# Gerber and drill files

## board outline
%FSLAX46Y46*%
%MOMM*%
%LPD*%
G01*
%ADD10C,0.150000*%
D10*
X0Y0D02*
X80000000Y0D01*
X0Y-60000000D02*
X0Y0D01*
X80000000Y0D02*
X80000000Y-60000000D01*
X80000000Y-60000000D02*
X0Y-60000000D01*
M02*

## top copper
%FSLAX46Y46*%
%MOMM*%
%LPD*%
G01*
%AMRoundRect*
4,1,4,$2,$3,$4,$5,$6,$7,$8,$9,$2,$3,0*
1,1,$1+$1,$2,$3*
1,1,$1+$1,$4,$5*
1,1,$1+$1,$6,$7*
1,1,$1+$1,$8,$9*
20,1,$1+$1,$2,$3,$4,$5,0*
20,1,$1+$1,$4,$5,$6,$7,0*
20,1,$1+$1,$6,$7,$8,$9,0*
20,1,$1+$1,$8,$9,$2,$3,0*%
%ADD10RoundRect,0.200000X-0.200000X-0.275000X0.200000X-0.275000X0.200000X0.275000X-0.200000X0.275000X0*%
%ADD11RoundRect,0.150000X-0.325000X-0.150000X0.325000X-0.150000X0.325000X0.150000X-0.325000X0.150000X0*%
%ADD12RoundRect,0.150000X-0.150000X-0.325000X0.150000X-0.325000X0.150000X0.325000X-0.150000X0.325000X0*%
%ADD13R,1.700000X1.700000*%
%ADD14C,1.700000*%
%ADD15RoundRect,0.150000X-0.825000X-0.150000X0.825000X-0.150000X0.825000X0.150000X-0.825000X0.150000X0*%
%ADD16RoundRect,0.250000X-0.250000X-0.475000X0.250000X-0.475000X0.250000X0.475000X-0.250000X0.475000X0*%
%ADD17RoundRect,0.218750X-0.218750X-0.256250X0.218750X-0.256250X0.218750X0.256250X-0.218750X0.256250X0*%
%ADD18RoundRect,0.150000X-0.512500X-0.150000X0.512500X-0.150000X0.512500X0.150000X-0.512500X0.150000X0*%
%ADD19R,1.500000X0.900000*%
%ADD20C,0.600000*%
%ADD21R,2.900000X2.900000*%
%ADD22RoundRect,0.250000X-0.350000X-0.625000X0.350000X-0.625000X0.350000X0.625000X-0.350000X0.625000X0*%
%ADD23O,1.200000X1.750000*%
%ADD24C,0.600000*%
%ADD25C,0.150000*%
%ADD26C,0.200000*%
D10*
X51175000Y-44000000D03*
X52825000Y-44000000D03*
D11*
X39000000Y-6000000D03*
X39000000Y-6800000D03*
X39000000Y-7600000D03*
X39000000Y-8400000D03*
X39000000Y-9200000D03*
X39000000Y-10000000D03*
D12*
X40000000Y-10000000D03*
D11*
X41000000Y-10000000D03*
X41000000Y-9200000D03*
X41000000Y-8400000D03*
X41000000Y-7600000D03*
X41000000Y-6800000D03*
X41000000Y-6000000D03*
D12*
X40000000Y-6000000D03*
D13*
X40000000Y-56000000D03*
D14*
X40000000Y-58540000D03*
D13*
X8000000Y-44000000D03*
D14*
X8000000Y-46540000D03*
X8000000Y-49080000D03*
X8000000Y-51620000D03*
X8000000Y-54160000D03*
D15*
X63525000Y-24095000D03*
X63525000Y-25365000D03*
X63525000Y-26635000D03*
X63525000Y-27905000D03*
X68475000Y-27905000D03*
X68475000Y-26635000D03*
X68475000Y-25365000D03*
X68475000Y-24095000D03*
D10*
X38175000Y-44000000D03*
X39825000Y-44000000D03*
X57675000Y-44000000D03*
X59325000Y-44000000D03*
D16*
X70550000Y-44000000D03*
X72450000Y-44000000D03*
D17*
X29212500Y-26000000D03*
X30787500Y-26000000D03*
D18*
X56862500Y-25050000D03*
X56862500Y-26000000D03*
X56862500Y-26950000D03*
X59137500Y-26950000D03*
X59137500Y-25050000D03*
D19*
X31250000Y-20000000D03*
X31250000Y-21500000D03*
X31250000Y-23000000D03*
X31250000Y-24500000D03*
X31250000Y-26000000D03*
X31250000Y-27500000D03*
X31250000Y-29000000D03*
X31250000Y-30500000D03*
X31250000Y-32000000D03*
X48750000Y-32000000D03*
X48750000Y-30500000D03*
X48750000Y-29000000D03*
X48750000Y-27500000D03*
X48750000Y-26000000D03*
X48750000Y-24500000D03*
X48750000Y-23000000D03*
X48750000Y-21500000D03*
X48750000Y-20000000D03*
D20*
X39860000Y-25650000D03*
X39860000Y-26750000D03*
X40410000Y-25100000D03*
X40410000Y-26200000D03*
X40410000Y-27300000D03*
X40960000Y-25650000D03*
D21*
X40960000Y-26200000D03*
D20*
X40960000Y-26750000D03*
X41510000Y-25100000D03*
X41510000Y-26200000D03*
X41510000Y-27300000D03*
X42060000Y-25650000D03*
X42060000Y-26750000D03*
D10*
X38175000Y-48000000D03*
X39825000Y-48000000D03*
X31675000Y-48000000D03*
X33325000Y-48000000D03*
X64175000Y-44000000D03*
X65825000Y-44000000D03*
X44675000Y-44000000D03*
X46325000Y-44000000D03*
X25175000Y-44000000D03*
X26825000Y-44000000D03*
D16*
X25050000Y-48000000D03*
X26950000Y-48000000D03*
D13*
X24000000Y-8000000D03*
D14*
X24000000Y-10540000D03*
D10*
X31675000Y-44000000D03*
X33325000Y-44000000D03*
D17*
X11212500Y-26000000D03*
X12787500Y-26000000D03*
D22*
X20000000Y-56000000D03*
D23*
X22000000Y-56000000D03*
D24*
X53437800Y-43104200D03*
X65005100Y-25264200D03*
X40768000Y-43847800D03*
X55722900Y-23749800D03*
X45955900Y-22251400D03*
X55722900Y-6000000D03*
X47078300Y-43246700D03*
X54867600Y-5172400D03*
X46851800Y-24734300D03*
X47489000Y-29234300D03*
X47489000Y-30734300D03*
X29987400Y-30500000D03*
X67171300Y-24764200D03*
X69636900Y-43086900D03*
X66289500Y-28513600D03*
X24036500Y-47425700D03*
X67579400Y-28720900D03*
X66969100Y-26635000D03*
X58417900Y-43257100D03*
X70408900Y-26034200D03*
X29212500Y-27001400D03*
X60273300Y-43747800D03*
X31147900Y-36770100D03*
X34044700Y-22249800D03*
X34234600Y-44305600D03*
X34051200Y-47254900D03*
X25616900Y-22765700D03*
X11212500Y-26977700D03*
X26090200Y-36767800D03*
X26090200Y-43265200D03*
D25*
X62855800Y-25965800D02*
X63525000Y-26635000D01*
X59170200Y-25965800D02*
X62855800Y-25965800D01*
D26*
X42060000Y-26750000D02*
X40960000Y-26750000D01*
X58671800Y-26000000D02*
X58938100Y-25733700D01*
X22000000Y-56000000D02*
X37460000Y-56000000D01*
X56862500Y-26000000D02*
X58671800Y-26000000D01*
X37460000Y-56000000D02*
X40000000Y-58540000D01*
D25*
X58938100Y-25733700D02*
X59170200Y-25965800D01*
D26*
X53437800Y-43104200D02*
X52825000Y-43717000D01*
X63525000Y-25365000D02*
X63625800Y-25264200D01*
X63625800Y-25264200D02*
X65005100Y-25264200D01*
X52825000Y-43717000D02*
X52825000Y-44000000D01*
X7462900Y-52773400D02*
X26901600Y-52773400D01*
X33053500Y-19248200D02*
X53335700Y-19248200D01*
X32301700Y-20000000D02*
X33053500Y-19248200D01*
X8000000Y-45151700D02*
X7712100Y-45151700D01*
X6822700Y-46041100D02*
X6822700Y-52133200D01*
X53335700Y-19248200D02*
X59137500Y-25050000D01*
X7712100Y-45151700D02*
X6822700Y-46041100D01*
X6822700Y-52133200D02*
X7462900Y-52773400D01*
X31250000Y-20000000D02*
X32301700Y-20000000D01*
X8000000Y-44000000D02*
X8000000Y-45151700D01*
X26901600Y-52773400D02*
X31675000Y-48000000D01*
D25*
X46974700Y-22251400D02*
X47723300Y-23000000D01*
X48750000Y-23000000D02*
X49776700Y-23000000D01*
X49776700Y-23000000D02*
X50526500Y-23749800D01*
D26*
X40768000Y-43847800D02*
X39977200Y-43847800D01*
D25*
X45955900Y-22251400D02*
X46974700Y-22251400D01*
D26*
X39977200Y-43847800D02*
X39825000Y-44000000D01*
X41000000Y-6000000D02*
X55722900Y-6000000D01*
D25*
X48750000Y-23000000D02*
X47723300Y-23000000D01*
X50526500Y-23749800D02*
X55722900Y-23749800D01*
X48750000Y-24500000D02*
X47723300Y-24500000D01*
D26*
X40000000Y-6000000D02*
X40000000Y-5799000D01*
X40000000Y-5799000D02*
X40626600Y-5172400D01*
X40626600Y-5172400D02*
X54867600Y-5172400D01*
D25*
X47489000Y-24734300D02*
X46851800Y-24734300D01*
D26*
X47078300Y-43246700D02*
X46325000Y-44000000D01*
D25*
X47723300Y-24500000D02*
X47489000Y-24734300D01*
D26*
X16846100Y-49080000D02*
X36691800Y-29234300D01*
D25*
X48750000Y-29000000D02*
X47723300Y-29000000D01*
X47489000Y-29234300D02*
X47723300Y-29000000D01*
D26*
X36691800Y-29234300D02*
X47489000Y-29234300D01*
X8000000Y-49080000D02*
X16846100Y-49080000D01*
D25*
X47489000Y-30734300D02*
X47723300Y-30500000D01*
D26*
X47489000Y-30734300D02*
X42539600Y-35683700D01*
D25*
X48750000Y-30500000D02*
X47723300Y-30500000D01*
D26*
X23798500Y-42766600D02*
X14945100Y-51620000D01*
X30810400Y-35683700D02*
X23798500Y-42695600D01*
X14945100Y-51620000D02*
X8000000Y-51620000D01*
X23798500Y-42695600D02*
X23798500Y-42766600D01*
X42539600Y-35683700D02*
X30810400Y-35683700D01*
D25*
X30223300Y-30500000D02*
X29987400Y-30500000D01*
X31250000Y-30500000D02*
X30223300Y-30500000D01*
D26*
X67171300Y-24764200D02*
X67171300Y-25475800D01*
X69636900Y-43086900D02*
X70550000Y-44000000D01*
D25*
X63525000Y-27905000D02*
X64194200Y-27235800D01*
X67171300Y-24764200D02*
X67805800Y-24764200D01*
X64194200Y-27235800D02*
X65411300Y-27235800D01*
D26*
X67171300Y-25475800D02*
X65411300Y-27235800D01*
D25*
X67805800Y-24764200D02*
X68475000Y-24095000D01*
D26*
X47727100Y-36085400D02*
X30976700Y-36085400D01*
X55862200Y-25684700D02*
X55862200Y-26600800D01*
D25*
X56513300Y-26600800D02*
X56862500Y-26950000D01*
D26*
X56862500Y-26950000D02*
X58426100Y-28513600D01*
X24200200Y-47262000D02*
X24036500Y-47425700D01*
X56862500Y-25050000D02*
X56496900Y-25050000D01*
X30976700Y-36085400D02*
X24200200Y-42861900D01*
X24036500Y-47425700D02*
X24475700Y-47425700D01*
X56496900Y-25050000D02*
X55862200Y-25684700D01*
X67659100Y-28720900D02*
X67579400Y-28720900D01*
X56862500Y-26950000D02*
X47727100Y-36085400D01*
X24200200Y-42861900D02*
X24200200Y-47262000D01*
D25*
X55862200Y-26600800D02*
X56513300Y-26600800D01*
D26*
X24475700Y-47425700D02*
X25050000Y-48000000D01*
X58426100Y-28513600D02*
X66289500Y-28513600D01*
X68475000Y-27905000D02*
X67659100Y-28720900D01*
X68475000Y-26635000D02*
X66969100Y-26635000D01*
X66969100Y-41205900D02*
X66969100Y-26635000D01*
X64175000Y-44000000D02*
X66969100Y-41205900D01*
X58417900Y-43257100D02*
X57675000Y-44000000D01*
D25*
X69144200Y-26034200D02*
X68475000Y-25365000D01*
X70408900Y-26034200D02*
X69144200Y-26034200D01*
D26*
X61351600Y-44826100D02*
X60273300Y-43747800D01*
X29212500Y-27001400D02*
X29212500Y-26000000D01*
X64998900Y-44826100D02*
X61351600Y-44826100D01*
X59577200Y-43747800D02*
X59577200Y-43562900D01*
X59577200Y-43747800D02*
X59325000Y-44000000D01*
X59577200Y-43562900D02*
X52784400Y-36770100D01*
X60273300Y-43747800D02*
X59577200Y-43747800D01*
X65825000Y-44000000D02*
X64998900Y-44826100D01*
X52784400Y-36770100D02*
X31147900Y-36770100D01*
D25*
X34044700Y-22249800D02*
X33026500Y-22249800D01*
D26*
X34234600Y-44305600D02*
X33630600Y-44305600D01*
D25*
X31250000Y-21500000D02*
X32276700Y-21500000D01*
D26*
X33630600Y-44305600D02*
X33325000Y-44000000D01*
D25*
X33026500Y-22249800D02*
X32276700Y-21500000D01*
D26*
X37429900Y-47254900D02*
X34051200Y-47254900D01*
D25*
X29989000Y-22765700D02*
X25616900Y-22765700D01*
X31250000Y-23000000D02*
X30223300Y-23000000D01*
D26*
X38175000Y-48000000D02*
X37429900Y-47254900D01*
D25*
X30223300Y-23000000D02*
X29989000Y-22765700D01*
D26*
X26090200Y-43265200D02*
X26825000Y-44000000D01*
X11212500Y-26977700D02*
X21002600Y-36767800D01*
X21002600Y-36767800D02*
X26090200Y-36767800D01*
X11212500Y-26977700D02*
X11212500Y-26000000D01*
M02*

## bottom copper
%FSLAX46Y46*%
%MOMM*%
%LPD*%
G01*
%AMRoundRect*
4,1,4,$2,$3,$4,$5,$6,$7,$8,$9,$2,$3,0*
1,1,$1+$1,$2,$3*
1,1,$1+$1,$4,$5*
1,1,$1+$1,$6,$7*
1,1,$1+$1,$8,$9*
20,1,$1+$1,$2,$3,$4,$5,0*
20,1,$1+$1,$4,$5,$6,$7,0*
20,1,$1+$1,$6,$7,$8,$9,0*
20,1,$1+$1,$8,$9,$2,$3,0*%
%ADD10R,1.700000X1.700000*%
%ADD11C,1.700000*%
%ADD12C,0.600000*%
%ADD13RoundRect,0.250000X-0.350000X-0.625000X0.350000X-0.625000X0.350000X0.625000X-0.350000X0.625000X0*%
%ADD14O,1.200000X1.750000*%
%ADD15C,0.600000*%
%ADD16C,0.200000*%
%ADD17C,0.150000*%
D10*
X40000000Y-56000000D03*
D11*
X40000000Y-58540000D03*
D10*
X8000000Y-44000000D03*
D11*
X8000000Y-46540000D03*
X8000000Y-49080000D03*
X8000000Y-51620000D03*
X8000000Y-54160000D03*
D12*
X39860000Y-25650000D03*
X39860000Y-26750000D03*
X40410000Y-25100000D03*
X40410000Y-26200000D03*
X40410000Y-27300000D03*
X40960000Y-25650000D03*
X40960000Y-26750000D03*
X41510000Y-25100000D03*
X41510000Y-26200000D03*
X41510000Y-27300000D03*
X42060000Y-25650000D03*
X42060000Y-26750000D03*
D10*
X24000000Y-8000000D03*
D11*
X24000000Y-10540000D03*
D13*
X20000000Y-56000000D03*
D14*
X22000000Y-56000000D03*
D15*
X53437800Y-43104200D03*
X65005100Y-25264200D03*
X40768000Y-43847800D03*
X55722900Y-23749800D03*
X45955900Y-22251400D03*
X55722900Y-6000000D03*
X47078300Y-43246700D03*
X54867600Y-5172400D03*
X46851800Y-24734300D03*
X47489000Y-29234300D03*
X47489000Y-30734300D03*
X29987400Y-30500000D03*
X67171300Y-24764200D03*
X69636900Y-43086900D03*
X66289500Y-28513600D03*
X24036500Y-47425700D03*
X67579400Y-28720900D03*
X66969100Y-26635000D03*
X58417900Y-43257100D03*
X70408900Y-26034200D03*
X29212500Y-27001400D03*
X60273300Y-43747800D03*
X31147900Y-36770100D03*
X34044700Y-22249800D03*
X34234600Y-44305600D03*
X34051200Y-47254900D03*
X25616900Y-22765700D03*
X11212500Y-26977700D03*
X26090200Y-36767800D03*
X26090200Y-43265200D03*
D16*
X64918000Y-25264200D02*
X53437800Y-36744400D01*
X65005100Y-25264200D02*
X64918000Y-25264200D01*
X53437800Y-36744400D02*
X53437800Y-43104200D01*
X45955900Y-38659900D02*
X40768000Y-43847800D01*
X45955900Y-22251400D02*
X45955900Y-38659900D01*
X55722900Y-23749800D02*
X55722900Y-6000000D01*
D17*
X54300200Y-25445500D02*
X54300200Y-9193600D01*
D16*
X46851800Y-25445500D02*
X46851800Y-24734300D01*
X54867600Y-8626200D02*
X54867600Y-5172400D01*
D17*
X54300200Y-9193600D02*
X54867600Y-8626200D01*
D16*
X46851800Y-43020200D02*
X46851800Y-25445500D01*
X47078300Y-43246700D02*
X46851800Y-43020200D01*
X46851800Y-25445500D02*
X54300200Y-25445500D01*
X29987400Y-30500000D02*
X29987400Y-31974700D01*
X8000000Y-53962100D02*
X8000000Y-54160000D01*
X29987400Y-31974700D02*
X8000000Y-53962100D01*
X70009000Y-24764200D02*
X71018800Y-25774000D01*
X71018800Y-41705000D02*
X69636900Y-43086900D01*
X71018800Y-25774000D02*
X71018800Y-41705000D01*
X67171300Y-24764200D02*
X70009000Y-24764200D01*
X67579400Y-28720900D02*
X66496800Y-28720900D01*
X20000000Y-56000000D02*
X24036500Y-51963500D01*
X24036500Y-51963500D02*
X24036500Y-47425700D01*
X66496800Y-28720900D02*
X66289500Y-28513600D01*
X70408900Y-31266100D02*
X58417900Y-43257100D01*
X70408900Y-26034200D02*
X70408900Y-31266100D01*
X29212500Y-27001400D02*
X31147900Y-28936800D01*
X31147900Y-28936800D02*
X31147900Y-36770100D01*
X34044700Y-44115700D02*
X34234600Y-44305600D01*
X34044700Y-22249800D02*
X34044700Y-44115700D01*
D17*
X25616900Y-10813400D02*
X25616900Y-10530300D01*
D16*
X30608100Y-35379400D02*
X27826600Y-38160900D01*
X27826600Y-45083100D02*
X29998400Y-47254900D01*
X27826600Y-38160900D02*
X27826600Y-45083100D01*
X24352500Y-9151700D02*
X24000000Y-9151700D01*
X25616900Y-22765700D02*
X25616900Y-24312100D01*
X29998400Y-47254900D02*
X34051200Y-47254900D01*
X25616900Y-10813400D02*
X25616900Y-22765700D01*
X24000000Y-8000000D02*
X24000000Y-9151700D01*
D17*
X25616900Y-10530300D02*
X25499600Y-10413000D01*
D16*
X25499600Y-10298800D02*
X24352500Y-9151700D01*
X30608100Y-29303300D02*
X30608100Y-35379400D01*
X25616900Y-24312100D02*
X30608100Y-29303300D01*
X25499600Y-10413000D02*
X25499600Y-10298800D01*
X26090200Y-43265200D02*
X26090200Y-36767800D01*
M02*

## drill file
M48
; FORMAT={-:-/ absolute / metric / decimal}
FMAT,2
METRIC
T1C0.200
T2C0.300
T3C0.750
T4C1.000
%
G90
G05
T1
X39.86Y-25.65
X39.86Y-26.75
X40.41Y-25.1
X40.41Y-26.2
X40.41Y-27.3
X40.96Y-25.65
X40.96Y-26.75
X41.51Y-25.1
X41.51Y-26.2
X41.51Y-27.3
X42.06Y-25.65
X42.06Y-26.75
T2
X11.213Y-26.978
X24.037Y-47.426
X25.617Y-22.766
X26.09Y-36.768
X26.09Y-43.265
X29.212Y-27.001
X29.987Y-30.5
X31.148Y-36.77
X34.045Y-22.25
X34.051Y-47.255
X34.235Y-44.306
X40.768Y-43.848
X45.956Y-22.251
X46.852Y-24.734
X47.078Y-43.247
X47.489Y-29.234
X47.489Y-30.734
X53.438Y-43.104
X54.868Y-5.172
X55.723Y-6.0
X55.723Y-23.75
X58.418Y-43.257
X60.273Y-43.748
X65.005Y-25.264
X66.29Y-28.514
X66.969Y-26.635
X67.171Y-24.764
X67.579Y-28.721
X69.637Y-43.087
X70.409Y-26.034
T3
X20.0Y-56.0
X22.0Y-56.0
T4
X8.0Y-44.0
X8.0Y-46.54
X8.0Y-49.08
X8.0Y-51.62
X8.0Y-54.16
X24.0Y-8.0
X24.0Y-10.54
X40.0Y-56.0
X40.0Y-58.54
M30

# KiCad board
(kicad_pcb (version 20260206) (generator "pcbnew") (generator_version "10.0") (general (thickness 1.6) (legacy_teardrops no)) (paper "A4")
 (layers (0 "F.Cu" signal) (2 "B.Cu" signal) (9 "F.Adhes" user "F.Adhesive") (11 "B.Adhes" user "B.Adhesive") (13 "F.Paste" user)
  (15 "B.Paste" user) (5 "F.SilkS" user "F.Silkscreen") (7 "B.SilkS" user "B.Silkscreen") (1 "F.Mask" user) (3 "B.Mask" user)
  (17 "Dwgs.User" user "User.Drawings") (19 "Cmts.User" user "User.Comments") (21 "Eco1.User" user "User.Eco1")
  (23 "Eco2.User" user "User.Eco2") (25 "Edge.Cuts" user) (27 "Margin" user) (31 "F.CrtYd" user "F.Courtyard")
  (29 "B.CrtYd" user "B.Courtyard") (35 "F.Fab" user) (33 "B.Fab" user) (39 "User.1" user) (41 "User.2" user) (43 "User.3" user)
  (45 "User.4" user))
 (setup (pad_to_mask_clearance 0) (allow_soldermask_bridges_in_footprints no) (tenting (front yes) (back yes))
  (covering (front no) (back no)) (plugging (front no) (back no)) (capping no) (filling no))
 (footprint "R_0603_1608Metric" (layer "F.Cu") (at 52 44)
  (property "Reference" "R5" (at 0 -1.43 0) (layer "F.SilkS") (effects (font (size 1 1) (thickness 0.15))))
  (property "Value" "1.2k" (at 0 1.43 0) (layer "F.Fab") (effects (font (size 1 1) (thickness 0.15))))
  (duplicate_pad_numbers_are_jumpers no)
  (pad "1" smd roundrect (at -0.825 0) (size 0.8 0.95) (layers "F.Cu" "F.Mask" "F.Paste") (roundrect_rratio 0.25) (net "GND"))
  (pad "2" smd roundrect (at 0.825 0) (size 0.8 0.95) (layers "F.Cu" "F.Mask" "F.Paste") (roundrect_rratio 0.25) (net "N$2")))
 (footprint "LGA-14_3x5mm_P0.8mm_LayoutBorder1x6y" (layer "F.Cu") (at 40 8)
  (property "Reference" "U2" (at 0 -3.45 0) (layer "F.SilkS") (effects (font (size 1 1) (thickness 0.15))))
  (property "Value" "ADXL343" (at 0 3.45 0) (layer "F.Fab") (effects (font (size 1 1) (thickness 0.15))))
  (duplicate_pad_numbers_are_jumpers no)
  (pad "1" smd roundrect (at -1 -2) (size 0.95 0.6) (layers "F.Cu" "F.Mask" "F.Paste") (roundrect_rratio 0.25) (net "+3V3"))
  (pad "2" smd roundrect (at -1 -1.2) (size 0.95 0.6) (layers "F.Cu" "F.Mask" "F.Paste") (roundrect_rratio 0.25) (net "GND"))
  (pad "3" smd roundrect (at -1 -0.4) (size 0.95 0.6) (layers "F.Cu" "F.Mask" "F.Paste") (roundrect_rratio 0.25))
  (pad "4" smd roundrect (at -1 0.4) (size 0.95 0.6) (layers "F.Cu" "F.Mask" "F.Paste") (roundrect_rratio 0.25) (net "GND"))
  (pad "5" smd roundrect (at -1 1.2) (size 0.95 0.6) (layers "F.Cu" "F.Mask" "F.Paste") (roundrect_rratio 0.25) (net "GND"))
  (pad "6" smd roundrect (at -1 2) (size 0.95 0.6) (layers "F.Cu" "F.Mask" "F.Paste") (roundrect_rratio 0.25) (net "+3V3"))
  (pad "7" smd roundrect (at 0 2) (size 0.6 0.95) (layers "F.Cu" "F.Mask" "F.Paste") (roundrect_rratio 0.25) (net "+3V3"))
  (pad "8" smd roundrect (at 1 2) (size 0.95 0.6) (layers "F.Cu" "F.Mask" "F.Paste") (roundrect_rratio 0.25) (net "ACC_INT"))
  (pad "9" smd roundrect (at 1 1.2) (size 0.95 0.6) (layers "F.Cu" "F.Mask" "F.Paste") (roundrect_rratio 0.25))
  (pad "10" smd roundrect (at 1 0.4) (size 0.95 0.6) (layers "F.Cu" "F.Mask" "F.Paste") (roundrect_rratio 0.25))
  (pad "11" smd roundrect (at 1 -0.4) (size 0.95 0.6) (layers "F.Cu" "F.Mask" "F.Paste") (roundrect_rratio 0.25))
  (pad "12" smd roundrect (at 1 -1.2) (size 0.95 0.6) (layers "F.Cu" "F.Mask" "F.Paste") (roundrect_rratio 0.25) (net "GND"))
  (pad "13" smd roundrect (at 1 -2) (size 0.95 0.6) (layers "F.Cu" "F.Mask" "F.Paste") (roundrect_rratio 0.25) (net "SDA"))
  (pad "14" smd roundrect (at 0 -2) (size 0.6 0.95) (layers "F.Cu" "F.Mask" "F.Paste") (roundrect_rratio 0.25) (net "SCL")))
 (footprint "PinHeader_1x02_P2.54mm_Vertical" (layer "F.Cu") (at 40 56)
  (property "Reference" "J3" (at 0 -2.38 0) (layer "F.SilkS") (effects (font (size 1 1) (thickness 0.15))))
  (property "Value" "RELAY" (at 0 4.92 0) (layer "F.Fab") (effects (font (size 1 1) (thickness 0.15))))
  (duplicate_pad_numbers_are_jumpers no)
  (pad "1" thru_hole rect (at 0 0) (size 1.7 1.7) (drill 1) (layers "*.Cu" "*.Mask") (remove_unused_layers no) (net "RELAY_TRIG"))
  (pad "2" thru_hole circle (at 0 2.54) (size 1.7 1.7) (drill 1) (layers "*.Cu" "*.Mask") (remove_unused_layers no) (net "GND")))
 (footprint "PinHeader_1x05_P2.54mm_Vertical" (layer "F.Cu") (at 8 44)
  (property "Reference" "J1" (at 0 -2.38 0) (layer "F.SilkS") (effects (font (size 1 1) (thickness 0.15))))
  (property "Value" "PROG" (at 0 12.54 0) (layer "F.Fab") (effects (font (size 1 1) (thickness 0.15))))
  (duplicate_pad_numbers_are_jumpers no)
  (pad "1" thru_hole rect (at 0 0) (size 1.7 1.7) (drill 1) (layers "*.Cu" "*.Mask") (remove_unused_layers no) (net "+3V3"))
  (pad "2" thru_hole circle (at 0 2.54) (size 1.7 1.7) (drill 1) (layers "*.Cu" "*.Mask") (remove_unused_layers no) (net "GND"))
  (pad "3" thru_hole circle (at 0 5.08) (size 1.7 1.7) (drill 1) (layers "*.Cu" "*.Mask") (remove_unused_layers no) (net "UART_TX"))
  (pad "4" thru_hole circle (at 0 7.62) (size 1.7 1.7) (drill 1) (layers "*.Cu" "*.Mask") (remove_unused_layers no) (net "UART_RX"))
  (pad "5" thru_hole circle (at 0 10.16) (size 1.7 1.7) (drill 1) (layers "*.Cu" "*.Mask") (remove_unused_layers no) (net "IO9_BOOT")))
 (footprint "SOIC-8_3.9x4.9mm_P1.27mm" (layer "F.Cu") (at 66 26)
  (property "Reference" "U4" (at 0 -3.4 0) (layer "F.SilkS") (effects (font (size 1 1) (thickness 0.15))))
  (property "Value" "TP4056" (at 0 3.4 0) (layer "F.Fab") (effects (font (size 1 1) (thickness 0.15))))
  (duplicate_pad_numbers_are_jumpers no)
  (pad "1" smd roundrect (at -2.475 -1.905) (size 1.95 0.6) (layers "F.Cu" "F.Mask" "F.Paste") (roundrect_rratio 0.25) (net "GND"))
  (pad "2" smd roundrect (at -2.475 -0.635) (size 1.95 0.6) (layers "F.Cu" "F.Mask" "F.Paste") (roundrect_rratio 0.25) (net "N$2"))
  (pad "3" smd roundrect (at -2.475 0.635) (size 1.95 0.6) (layers "F.Cu" "F.Mask" "F.Paste") (roundrect_rratio 0.25) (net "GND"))
  (pad "4" smd roundrect (at -2.475 1.905) (size 1.95 0.6) (layers "F.Cu" "F.Mask" "F.Paste") (roundrect_rratio 0.25) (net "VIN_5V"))
  (pad "5" smd roundrect (at 2.475 1.905) (size 1.95 0.6) (layers "F.Cu" "F.Mask" "F.Paste") (roundrect_rratio 0.25) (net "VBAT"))
  (pad "6" smd roundrect (at 2.475 0.635) (size 1.95 0.6) (layers "F.Cu" "F.Mask" "F.Paste") (roundrect_rratio 0.25) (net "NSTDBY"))
  (pad "7" smd roundrect (at 2.475 -0.635) (size 1.95 0.6) (layers "F.Cu" "F.Mask" "F.Paste") (roundrect_rratio 0.25) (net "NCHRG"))
  (pad "8" smd roundrect (at 2.475 -1.905) (size 1.95 0.6) (layers "F.Cu" "F.Mask" "F.Paste") (roundrect_rratio 0.25) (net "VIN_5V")))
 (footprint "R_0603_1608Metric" (layer "F.Cu") (at 39 44)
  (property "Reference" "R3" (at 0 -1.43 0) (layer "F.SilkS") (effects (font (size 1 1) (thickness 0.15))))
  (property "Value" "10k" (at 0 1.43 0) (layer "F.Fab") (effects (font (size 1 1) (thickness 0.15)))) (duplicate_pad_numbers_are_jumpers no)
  (pad "1" smd roundrect (at -0.825 0) (size 0.8 0.95) (layers "F.Cu" "F.Mask" "F.Paste") (roundrect_rratio 0.25) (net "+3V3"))
  (pad "2" smd roundrect (at 0.825 0) (size 0.8 0.95) (layers "F.Cu" "F.Mask" "F.Paste") (roundrect_rratio 0.25) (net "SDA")))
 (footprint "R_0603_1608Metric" (layer "F.Cu") (at 58.5 44)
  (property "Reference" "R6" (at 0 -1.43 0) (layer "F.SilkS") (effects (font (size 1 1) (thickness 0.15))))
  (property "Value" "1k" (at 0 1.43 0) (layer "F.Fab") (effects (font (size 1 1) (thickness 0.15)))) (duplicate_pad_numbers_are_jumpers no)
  (pad "1" smd roundrect (at -0.825 0) (size 0.8 0.95) (layers "F.Cu" "F.Mask" "F.Paste") (roundrect_rratio 0.25) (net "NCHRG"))
  (pad "2" smd roundrect (at 0.825 0) (size 0.8 0.95) (layers "F.Cu" "F.Mask" "F.Paste") (roundrect_rratio 0.25) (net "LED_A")))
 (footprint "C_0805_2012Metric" (layer "F.Cu") (at 71.5 44)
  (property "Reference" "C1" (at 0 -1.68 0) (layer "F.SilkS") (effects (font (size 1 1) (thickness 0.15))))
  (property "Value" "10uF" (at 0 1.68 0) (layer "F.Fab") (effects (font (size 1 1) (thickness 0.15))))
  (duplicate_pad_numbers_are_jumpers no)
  (pad "1" smd roundrect (at -0.95 0) (size 1 1.45) (layers "F.Cu" "F.Mask" "F.Paste") (roundrect_rratio 0.25) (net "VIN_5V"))
  (pad "2" smd roundrect (at 0.95 0) (size 1 1.45) (layers "F.Cu" "F.Mask" "F.Paste") (roundrect_rratio 0.25) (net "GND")))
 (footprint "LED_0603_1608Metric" (layer "F.Cu") (at 30 26)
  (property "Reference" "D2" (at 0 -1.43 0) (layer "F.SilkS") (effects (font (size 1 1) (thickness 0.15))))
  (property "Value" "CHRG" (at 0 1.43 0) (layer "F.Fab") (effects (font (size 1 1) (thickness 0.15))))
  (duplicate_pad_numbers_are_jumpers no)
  (pad "1" smd roundrect (at -0.7875 0) (size 0.875 0.95) (layers "F.Cu" "F.Mask" "F.Paste") (roundrect_rratio 0.25) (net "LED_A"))
  (pad "2" smd roundrect (at 0.7875 0) (size 0.875 0.95) (layers "F.Cu" "F.Mask" "F.Paste") (roundrect_rratio 0.25) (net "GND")))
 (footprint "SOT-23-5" (layer "F.Cu") (at 58 26)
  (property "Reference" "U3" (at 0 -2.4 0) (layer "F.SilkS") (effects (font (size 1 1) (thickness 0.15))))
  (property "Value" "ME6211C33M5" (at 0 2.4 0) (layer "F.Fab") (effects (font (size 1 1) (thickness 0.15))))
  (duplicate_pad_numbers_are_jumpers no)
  (pad "1" smd roundrect (at -1.1375 -0.95) (size 1.325 0.6) (layers "F.Cu" "F.Mask" "F.Paste") (roundrect_rratio 0.25) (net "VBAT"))
  (pad "2" smd roundrect (at -1.1375 0) (size 1.325 0.6) (layers "F.Cu" "F.Mask" "F.Paste") (roundrect_rratio 0.25) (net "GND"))
  (pad "3" smd roundrect (at -1.1375 0.95) (size 1.325 0.6) (layers "F.Cu" "F.Mask" "F.Paste") (roundrect_rratio 0.25) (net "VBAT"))
  (pad "4" smd roundrect (at 1.1375 0.95) (size 1.325 0.6) (layers "F.Cu" "F.Mask" "F.Paste") (roundrect_rratio 0.25))
  (pad "5" smd roundrect (at 1.1375 -0.95) (size 1.325 0.6) (layers "F.Cu" "F.Mask" "F.Paste") (roundrect_rratio 0.25) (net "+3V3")))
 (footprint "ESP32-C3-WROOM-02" (layer "F.Cu") (at 40 26)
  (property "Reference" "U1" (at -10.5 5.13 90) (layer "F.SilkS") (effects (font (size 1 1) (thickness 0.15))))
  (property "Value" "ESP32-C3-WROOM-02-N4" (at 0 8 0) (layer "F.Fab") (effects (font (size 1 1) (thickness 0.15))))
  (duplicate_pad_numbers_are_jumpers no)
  (pad "" smd rect (at -0.14 -0.9) (size 0.7 0.7) (layers "F.Paste"))
  (pad "" smd rect (at -0.14 0.2) (size 0.7 0.7) (layers "F.Paste"))
  (pad "" smd rect (at -0.14 1.3) (size 0.7 0.7) (layers "F.Paste"))
  (pad "" smd rect (at 0.96 -0.9) (size 0.7 0.7) (layers "F.Paste"))
  (pad "" smd rect (at 0.96 0.2) (size 0.7 0.7) (layers "F.Paste"))
  (pad "" smd rect (at 0.96 1.3) (size 0.7 0.7) (layers "F.Paste"))
  (pad "" smd rect (at 2.06 -0.9) (size 0.7 0.7) (layers "F.Paste"))
  (pad "" smd rect (at 2.06 0.2) (size 0.7 0.7) (layers "F.Paste"))
  (pad "" smd rect (at 2.06 1.3) (size 0.7 0.7) (layers "F.Paste"))
  (pad "1" smd rect (at -8.75 -6) (size 1.5 0.9) (layers "F.Cu" "F.Mask" "F.Paste") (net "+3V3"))
  (pad "2" smd rect (at -8.75 -4.5) (size 1.5 0.9) (layers "F.Cu" "F.Mask" "F.Paste") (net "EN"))
  (pad "3" smd rect (at -8.75 -3) (size 1.5 0.9) (layers "F.Cu" "F.Mask" "F.Paste") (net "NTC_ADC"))
  (pad "4" smd rect (at -8.75 -1.5) (size 1.5 0.9) (layers "F.Cu" "F.Mask" "F.Paste") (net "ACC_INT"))
  (pad "5" smd rect (at -8.75 0) (size 1.5 0.9) (layers "F.Cu" "F.Mask" "F.Paste") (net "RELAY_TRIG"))
  (pad "6" smd rect (at -8.75 1.5) (size 1.5 0.9) (layers "F.Cu" "F.Mask" "F.Paste"))
  (pad "7" smd rect (at -8.75 3) (size 1.5 0.9) (layers "F.Cu" "F.Mask" "F.Paste"))
  (pad "8" smd rect (at -8.75 4.5) (size 1.5 0.9) (layers "F.Cu" "F.Mask" "F.Paste") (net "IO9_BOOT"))
  (pad "9" smd rect (at -8.75 6) (size 1.5 0.9) (layers "F.Cu" "F.Mask" "F.Paste") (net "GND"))
  (pad "10" smd rect (at 8.75 6) (size 1.5 0.9) (layers "F.Cu" "F.Mask" "F.Paste"))
  (pad "11" smd rect (at 8.75 4.5) (size 1.5 0.9) (layers "F.Cu" "F.Mask" "F.Paste") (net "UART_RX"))
  (pad "12" smd rect (at 8.75 3) (size 1.5 0.9) (layers "F.Cu" "F.Mask" "F.Paste") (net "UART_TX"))
  (pad "13" smd rect (at 8.75 1.5) (size 1.5 0.9) (layers "F.Cu" "F.Mask" "F.Paste"))
  (pad "14" smd rect (at 8.75 0) (size 1.5 0.9) (layers "F.Cu" "F.Mask" "F.Paste"))
  (pad "15" smd rect (at 8.75 -1.5) (size 1.5 0.9) (layers "F.Cu" "F.Mask" "F.Paste") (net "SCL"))
  (pad "16" smd rect (at 8.75 -3) (size 1.5 0.9) (layers "F.Cu" "F.Mask" "F.Paste") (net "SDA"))
  (pad "17" smd rect (at 8.75 -4.5) (size 1.5 0.9) (layers "F.Cu" "F.Mask" "F.Paste"))
  (pad "18" smd rect (at 8.75 -6) (size 1.5 0.9) (layers "F.Cu" "F.Mask" "F.Paste"))
  (pad "19" thru_hole circle (at -0.14 -0.35) (size 0.6 0.6) (drill 0.2) (layers "*.Cu" "F.Mask") (remove_unused_layers no) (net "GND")
   (zone_connect 2))
  (pad "19" thru_hole circle (at -0.14 0.75) (size 0.6 0.6) (drill 0.2) (layers "*.Cu" "F.Mask") (remove_unused_layers no) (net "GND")
   (zone_connect 2))
  (pad "19" thru_hole circle (at 0.41 -0.9) (size 0.6 0.6) (drill 0.2) (layers "*.Cu" "F.Mask") (remove_unused_layers no) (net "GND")
   (zone_connect 2))
  (pad "19" thru_hole circle (at 0.41 0.2) (size 0.6 0.6) (drill 0.2) (layers "*.Cu" "F.Mask") (remove_unused_layers no) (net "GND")
   (zone_connect 2))
  (pad "19" thru_hole circle (at 0.41 1.3) (size 0.6 0.6) (drill 0.2) (layers "*.Cu" "F.Mask") (remove_unused_layers no) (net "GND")
   (zone_connect 2))
  (pad "19" thru_hole circle (at 0.96 -0.35) (size 0.6 0.6) (drill 0.2) (layers "*.Cu" "F.Mask") (remove_unused_layers no) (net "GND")
   (zone_connect 2))
  (pad "19" smd rect (at 0.96 0.2) (size 2.9 2.9) (layers "F.Cu" "F.Mask") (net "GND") (zone_connect 2))
  (pad "19" thru_hole circle (at 0.96 0.75) (size 0.6 0.6) (drill 0.2) (layers "*.Cu" "F.Mask") (remove_unused_layers no) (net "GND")
   (zone_connect 2))
  (pad "19" thru_hole circle (at 1.51 -0.9) (size 0.6 0.6) (drill 0.2) (layers "*.Cu" "F.Mask") (remove_unused_layers no) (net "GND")
   (zone_connect 2))
  (pad "19" thru_hole circle (at 1.51 0.2) (size 0.6 0.6) (drill 0.2) (layers "*.Cu" "F.Mask") (remove_unused_layers no) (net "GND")
   (zone_connect 2))
  (pad "19" thru_hole circle (at 1.51 1.3) (size 0.6 0.6) (drill 0.2) (layers "*.Cu" "F.Mask") (remove_unused_layers no) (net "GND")
   (zone_connect 2))
  (pad "19" thru_hole circle (at 2.06 -0.35) (size 0.6 0.6) (drill 0.2) (layers "*.Cu" "F.Mask") (remove_unused_layers no) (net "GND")
   (zone_connect 2))
  (pad "19" thru_hole circle (at 2.06 0.75) (size 0.6 0.6) (drill 0.2) (layers "*.Cu" "F.Mask") (remove_unused_layers no) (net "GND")
   (zone_connect 2))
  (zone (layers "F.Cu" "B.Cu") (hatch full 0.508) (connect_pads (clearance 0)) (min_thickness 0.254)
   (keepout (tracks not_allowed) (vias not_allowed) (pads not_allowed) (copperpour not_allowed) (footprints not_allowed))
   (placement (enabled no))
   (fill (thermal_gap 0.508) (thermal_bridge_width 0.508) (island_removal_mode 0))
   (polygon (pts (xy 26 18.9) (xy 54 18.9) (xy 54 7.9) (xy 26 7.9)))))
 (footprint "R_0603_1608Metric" (layer "F.Cu") (at 39 48)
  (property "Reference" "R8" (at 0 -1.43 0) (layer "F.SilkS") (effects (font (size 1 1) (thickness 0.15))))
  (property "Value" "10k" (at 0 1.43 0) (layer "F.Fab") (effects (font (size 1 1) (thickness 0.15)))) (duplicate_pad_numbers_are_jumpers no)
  (pad "1" smd roundrect (at -0.825 0) (size 0.8 0.95) (layers "F.Cu" "F.Mask" "F.Paste") (roundrect_rratio 0.25) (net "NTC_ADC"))
  (pad "2" smd roundrect (at 0.825 0) (size 0.8 0.95) (layers "F.Cu" "F.Mask" "F.Paste") (roundrect_rratio 0.25) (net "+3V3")))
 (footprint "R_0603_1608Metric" (layer "F.Cu") (at 32.5 48)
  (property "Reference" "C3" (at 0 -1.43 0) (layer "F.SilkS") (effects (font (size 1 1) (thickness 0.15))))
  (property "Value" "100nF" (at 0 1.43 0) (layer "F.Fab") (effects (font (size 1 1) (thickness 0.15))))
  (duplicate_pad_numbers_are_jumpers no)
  (pad "1" smd roundrect (at -0.825 0) (size 0.8 0.95) (layers "F.Cu" "F.Mask" "F.Paste") (roundrect_rratio 0.25) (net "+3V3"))
  (pad "2" smd roundrect (at 0.825 0) (size 0.8 0.95) (layers "F.Cu" "F.Mask" "F.Paste") (roundrect_rratio 0.25) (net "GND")))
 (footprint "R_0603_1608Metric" (layer "F.Cu") (at 65 44)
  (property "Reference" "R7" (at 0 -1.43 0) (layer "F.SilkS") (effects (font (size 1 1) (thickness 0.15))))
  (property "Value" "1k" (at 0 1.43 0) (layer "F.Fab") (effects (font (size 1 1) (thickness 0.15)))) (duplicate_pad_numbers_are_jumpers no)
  (pad "1" smd roundrect (at -0.825 0) (size 0.8 0.95) (layers "F.Cu" "F.Mask" "F.Paste") (roundrect_rratio 0.25) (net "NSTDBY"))
  (pad "2" smd roundrect (at 0.825 0) (size 0.8 0.95) (layers "F.Cu" "F.Mask" "F.Paste") (roundrect_rratio 0.25) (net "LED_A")))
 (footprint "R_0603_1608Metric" (layer "F.Cu") (at 45.5 44)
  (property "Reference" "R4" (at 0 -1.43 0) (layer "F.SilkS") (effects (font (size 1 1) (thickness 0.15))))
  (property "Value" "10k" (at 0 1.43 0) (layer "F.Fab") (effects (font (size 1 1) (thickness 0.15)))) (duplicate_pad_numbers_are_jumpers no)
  (pad "1" smd roundrect (at -0.825 0) (size 0.8 0.95) (layers "F.Cu" "F.Mask" "F.Paste") (roundrect_rratio 0.25) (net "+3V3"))
  (pad "2" smd roundrect (at 0.825 0) (size 0.8 0.95) (layers "F.Cu" "F.Mask" "F.Paste") (roundrect_rratio 0.25) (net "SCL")))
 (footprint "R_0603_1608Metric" (layer "F.Cu") (at 26 44)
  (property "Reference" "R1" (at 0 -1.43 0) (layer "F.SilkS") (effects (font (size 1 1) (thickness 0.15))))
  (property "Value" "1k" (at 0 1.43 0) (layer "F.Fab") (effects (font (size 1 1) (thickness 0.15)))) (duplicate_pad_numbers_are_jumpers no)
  (pad "1" smd roundrect (at -0.825 0) (size 0.8 0.95) (layers "F.Cu" "F.Mask" "F.Paste") (roundrect_rratio 0.25) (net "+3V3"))
  (pad "2" smd roundrect (at 0.825 0) (size 0.8 0.95) (layers "F.Cu" "F.Mask" "F.Paste") (roundrect_rratio 0.25) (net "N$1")))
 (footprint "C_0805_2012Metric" (layer "F.Cu") (at 26 48)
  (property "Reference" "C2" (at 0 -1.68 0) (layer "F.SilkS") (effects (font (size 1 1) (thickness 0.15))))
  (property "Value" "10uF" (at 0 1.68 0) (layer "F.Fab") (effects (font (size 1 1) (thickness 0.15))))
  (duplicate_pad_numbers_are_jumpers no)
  (pad "1" smd roundrect (at -0.95 0) (size 1 1.45) (layers "F.Cu" "F.Mask" "F.Paste") (roundrect_rratio 0.25) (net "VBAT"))
  (pad "2" smd roundrect (at 0.95 0) (size 1 1.45) (layers "F.Cu" "F.Mask" "F.Paste") (roundrect_rratio 0.25) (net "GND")))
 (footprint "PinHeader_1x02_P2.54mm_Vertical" (layer "F.Cu") (at 24 8)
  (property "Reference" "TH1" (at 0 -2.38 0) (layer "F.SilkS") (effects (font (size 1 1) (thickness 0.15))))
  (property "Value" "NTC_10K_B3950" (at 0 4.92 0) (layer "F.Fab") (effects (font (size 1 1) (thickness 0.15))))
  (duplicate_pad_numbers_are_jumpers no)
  (pad "1" thru_hole rect (at 0 0) (size 1.7 1.7) (drill 1) (layers "*.Cu" "*.Mask") (remove_unused_layers no) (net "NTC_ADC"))
  (pad "2" thru_hole circle (at 0 2.54) (size 1.7 1.7) (drill 1) (layers "*.Cu" "*.Mask") (remove_unused_layers no) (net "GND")))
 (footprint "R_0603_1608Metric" (layer "F.Cu") (at 32.5 44)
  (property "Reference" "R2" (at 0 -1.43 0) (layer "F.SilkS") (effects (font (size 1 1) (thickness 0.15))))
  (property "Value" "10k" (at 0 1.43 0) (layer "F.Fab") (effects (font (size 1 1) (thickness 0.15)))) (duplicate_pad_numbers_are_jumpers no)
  (pad "1" smd roundrect (at -0.825 0) (size 0.8 0.95) (layers "F.Cu" "F.Mask" "F.Paste") (roundrect_rratio 0.25) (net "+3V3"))
  (pad "2" smd roundrect (at 0.825 0) (size 0.8 0.95) (layers "F.Cu" "F.Mask" "F.Paste") (roundrect_rratio 0.25) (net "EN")))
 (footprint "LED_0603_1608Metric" (layer "F.Cu") (at 12 26)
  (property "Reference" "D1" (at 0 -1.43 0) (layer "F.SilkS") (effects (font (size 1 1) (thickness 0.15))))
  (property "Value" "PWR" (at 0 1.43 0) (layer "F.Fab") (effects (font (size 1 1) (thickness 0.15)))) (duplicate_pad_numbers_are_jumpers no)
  (pad "1" smd roundrect (at -0.7875 0) (size 0.875 0.95) (layers "F.Cu" "F.Mask" "F.Paste") (roundrect_rratio 0.25) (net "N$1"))
  (pad "2" smd roundrect (at 0.7875 0) (size 0.875 0.95) (layers "F.Cu" "F.Mask" "F.Paste") (roundrect_rratio 0.25) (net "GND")))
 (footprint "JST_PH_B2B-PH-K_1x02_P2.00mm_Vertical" (layer "F.Cu") (at 20 56)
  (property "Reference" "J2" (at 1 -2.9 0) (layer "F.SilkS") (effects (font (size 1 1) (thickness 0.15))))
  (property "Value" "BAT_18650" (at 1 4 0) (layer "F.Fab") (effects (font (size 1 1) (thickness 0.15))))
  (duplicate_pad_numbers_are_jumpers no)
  (pad "1" thru_hole roundrect (at 0 0) (size 1.2 1.75) (drill 0.75) (layers "*.Cu" "*.Mask") (remove_unused_layers no)
   (roundrect_rratio 0.208333) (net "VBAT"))
  (pad "2" thru_hole oval (at 2 0) (size 1.2 1.75) (drill 0.75) (layers "*.Cu" "*.Mask") (remove_unused_layers no) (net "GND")))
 (gr_line (start 0 0) (end 80 0) (stroke (width 0.15) (type default)) (layer "Edge.Cuts"))
 (gr_line (start 0 60) (end 0 0) (stroke (width 0.15) (type default)) (layer "Edge.Cuts"))
 (gr_line (start 80 0) (end 80 60) (stroke (width 0.15) (type default)) (layer "Edge.Cuts"))
 (gr_line (start 80 60) (end 0 60) (stroke (width 0.15) (type default)) (layer "Edge.Cuts"))
 (segment (start 62.8558 25.9658) (end 63.525 26.635) (width 0.15) (layer "F.Cu") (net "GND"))
 (segment (start 59.1702 25.9658) (end 62.8558 25.9658) (width 0.15) (layer "F.Cu") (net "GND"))
 (segment (start 42.06 26.75) (end 40.96 26.75) (width 0.2) (layer "F.Cu") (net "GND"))
 (segment (start 58.6718 26) (end 58.9381 25.7337) (width 0.2) (layer "F.Cu") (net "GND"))
 (segment (start 22 56) (end 37.46 56) (width 0.2) (layer "F.Cu") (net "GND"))
 (segment (start 56.8625 26) (end 58.6718 26) (width 0.2) (layer "F.Cu") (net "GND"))
 (segment (start 37.46 56) (end 40 58.54) (width 0.2) (layer "F.Cu") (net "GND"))
 (segment (start 58.9381 25.7337) (end 59.1702 25.9658) (width 0.15) (layer "F.Cu") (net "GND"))
 (segment (start 53.4378 43.1042) (end 52.825 43.717) (width 0.2) (layer "F.Cu") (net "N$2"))
 (segment (start 63.525 25.365) (end 63.6258 25.2642) (width 0.2) (layer "F.Cu") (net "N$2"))
 (segment (start 63.6258 25.2642) (end 65.0051 25.2642) (width 0.2) (layer "F.Cu") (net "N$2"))
 (segment (start 52.825 43.717) (end 52.825 44) (width 0.2) (layer "F.Cu") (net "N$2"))
 (via (at 53.4378 43.1042) (size 0.6) (drill 0.3) (layers "F.Cu" "B.Cu") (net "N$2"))
 (via (at 65.0051 25.2642) (size 0.6) (drill 0.3) (layers "F.Cu" "B.Cu") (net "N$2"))
 (segment (start 64.918 25.2642) (end 53.4378 36.7444) (width 0.2) (layer "B.Cu") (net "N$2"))
 (segment (start 65.0051 25.2642) (end 64.918 25.2642) (width 0.2) (layer "B.Cu") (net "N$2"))
 (segment (start 53.4378 36.7444) (end 53.4378 43.1042) (width 0.2) (layer "B.Cu") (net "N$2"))
 (segment (start 7.4629 52.7734) (end 26.9016 52.7734) (width 0.2) (layer "F.Cu") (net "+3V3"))
 (segment (start 33.0535 19.2482) (end 53.3357 19.2482) (width 0.2) (layer "F.Cu") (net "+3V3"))
 (segment (start 32.3017 20) (end 33.0535 19.2482) (width 0.2) (layer "F.Cu") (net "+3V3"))
 (segment (start 8 45.1517) (end 7.7121 45.1517) (width 0.2) (layer "F.Cu") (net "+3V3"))
 (segment (start 6.8227 46.0411) (end 6.8227 52.1332) (width 0.2) (layer "F.Cu") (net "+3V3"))
 (segment (start 53.3357 19.2482) (end 59.1375 25.05) (width 0.2) (layer "F.Cu") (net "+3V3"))
 (segment (start 7.7121 45.1517) (end 6.8227 46.0411) (width 0.2) (layer "F.Cu") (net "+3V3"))
 (segment (start 6.8227 52.1332) (end 7.4629 52.7734) (width 0.2) (layer "F.Cu") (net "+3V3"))
 (segment (start 31.25 20) (end 32.3017 20) (width 0.2) (layer "F.Cu") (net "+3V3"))
 (segment (start 8 44) (end 8 45.1517) (width 0.2) (layer "F.Cu") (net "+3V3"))
 (segment (start 26.9016 52.7734) (end 31.675 48) (width 0.2) (layer "F.Cu") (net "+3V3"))
 (segment (start 46.9747 22.2514) (end 47.7233 23) (width 0.15) (layer "F.Cu") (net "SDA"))
 (segment (start 48.75 23) (end 49.7767 23) (width 0.15) (layer "F.Cu") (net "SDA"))
 (segment (start 49.7767 23) (end 50.5265 23.7498) (width 0.15) (layer "F.Cu") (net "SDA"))
 (segment (start 40.768 43.8478) (end 39.9772 43.8478) (width 0.2) (layer "F.Cu") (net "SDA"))
 (segment (start 45.9559 22.2514) (end 46.9747 22.2514) (width 0.15) (layer "F.Cu") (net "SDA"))
 (segment (start 39.9772 43.8478) (end 39.825 44) (width 0.2) (layer "F.Cu") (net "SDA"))
 (segment (start 41 6) (end 55.7229 6) (width 0.2) (layer "F.Cu") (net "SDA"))
 (segment (start 48.75 23) (end 47.7233 23) (width 0.15) (layer "F.Cu") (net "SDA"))
 (segment (start 50.5265 23.7498) (end 55.7229 23.7498) (width 0.15) (layer "F.Cu") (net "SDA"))
 (via (at 40.768 43.8478) (size 0.6) (drill 0.3) (layers "F.Cu" "B.Cu") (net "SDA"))
 (via (at 55.7229 23.7498) (size 0.6) (drill 0.3) (layers "F.Cu" "B.Cu") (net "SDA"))
 (via (at 45.9559 22.2514) (size 0.6) (drill 0.3) (layers "F.Cu" "B.Cu") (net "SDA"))
 (via (at 55.7229 6) (size 0.6) (drill 0.3) (layers "F.Cu" "B.Cu") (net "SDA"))
 (segment (start 45.9559 38.6599) (end 40.768 43.8478) (width 0.2) (layer "B.Cu") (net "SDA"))
 (segment (start 45.9559 22.2514) (end 45.9559 38.6599) (width 0.2) (layer "B.Cu") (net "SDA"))
 (segment (start 55.7229 23.7498) (end 55.7229 6) (width 0.2) (layer "B.Cu") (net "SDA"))
 (segment (start 48.75 24.5) (end 47.7233 24.5) (width 0.15) (layer "F.Cu") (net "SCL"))
 (segment (start 40 6) (end 40 5.799) (width 0.2) (layer "F.Cu") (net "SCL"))
 (segment (start 40 5.799) (end 40.6266 5.1724) (width 0.2) (layer "F.Cu") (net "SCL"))
 (segment (start 40.6266 5.1724) (end 54.8676 5.1724) (width 0.2) (layer "F.Cu") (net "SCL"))
 (segment (start 47.489 24.7343) (end 46.8518 24.7343) (width 0.15) (layer "F.Cu") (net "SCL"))
 (segment (start 47.0783 43.2467) (end 46.325 44) (width 0.2) (layer "F.Cu") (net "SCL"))
 (segment (start 47.7233 24.5) (end 47.489 24.7343) (width 0.15) (layer "F.Cu") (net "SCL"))
 (via (at 47.0783 43.2467) (size 0.6) (drill 0.3) (layers "F.Cu" "B.Cu") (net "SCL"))
 (via (at 54.8676 5.1724) (size 0.6) (drill 0.3) (layers "F.Cu" "B.Cu") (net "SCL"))
 (via (at 46.8518 24.7343) (size 0.6) (drill 0.3) (layers "F.Cu" "B.Cu") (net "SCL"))
 (segment (start 54.3002 25.4455) (end 54.3002 9.1936) (width 0.15) (layer "B.Cu") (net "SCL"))
 (segment (start 46.8518 25.4455) (end 46.8518 24.7343) (width 0.2) (layer "B.Cu") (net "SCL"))
 (segment (start 54.8676 8.6262) (end 54.8676 5.1724) (width 0.2) (layer "B.Cu") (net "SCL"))
 (segment (start 54.3002 9.1936) (end 54.8676 8.6262) (width 0.15) (layer "B.Cu") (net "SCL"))
 (segment (start 46.8518 43.0202) (end 46.8518 25.4455) (width 0.2) (layer "B.Cu") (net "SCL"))
 (segment (start 47.0783 43.2467) (end 46.8518 43.0202) (width 0.2) (layer "B.Cu") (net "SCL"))
 (segment (start 46.8518 25.4455) (end 54.3002 25.4455) (width 0.2) (layer "B.Cu") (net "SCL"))
 (segment (start 16.8461 49.08) (end 36.6918 29.2343) (width 0.2) (layer "F.Cu") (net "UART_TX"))
 (segment (start 48.75 29) (end 47.7233 29) (width 0.15) (layer "F.Cu") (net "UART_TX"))
 (segment (start 47.489 29.2343) (end 47.7233 29) (width 0.15) (layer "F.Cu") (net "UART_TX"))
 (segment (start 36.6918 29.2343) (end 47.489 29.2343) (width 0.2) (layer "F.Cu") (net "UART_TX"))
 (segment (start 8 49.08) (end 16.8461 49.08) (width 0.2) (layer "F.Cu") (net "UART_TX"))
 (via (at 47.489 29.2343) (size 0.6) (drill 0.3) (layers "F.Cu" "B.Cu") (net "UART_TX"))
 (segment (start 47.489 30.7343) (end 47.7233 30.5) (width 0.15) (layer "F.Cu") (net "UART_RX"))
 (segment (start 47.489 30.7343) (end 42.5396 35.6837) (width 0.2) (layer "F.Cu") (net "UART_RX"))
 (segment (start 48.75 30.5) (end 47.7233 30.5) (width 0.15) (layer "F.Cu") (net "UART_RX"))
 (segment (start 23.7985 42.7666) (end 14.9451 51.62) (width 0.2) (layer "F.Cu") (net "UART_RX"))
 (segment (start 30.8104 35.6837) (end 23.7985 42.6956) (width 0.2) (layer "F.Cu") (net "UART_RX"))
 (segment (start 14.9451 51.62) (end 8 51.62) (width 0.2) (layer "F.Cu") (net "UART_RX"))
 (segment (start 23.7985 42.6956) (end 23.7985 42.7666) (width 0.2) (layer "F.Cu") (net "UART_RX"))
 (segment (start 42.5396 35.6837) (end 30.8104 35.6837) (width 0.2) (layer "F.Cu") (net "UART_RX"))
 (via (at 47.489 30.7343) (size 0.6) (drill 0.3) (layers "F.Cu" "B.Cu") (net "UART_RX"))
 (segment (start 30.2233 30.5) (end 29.9874 30.5) (width 0.15) (layer "F.Cu") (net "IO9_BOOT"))
 (segment (start 31.25 30.5) (end 30.2233 30.5) (width 0.15) (layer "F.Cu") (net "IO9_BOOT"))
 (via (at 29.9874 30.5) (size 0.6) (drill 0.3) (layers "F.Cu" "B.Cu") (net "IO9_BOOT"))
 (segment (start 29.9874 30.5) (end 29.9874 31.9747) (width 0.2) (layer "B.Cu") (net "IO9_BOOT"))
 (segment (start 8 53.9621) (end 8 54.16) (width 0.2) (layer "B.Cu") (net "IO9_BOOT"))
 (segment (start 29.9874 31.9747) (end 8 53.9621) (width 0.2) (layer "B.Cu") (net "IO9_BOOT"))
 (segment (start 67.1713 24.7642) (end 67.1713 25.4758) (width 0.2) (layer "F.Cu") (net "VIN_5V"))
 (segment (start 69.6369 43.0869) (end 70.55 44) (width 0.2) (layer "F.Cu") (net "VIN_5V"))
 (segment (start 63.525 27.905) (end 64.1942 27.2358) (width 0.15) (layer "F.Cu") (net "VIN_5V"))
 (segment (start 67.1713 24.7642) (end 67.8058 24.7642) (width 0.15) (layer "F.Cu") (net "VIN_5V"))
 (segment (start 64.1942 27.2358) (end 65.4113 27.2358) (width 0.15) (layer "F.Cu") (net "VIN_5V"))
 (segment (start 67.1713 25.4758) (end 65.4113 27.2358) (width 0.2) (layer "F.Cu") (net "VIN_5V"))
 (segment (start 67.8058 24.7642) (end 68.475 24.095) (width 0.15) (layer "F.Cu") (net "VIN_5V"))
 (via (at 67.1713 24.7642) (size 0.6) (drill 0.3) (layers "F.Cu" "B.Cu") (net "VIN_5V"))
 (via (at 69.6369 43.0869) (size 0.6) (drill 0.3) (layers "F.Cu" "B.Cu") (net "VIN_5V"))
 (segment (start 70.009 24.7642) (end 71.0188 25.774) (width 0.2) (layer "B.Cu") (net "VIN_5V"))
 (segment (start 71.0188 41.705) (end 69.6369 43.0869) (width 0.2) (layer "B.Cu") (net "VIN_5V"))
 (segment (start 71.0188 25.774) (end 71.0188 41.705) (width 0.2) (layer "B.Cu") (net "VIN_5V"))
 (segment (start 67.1713 24.7642) (end 70.009 24.7642) (width 0.2) (layer "B.Cu") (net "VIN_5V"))
 (segment (start 47.7271 36.0854) (end 30.9767 36.0854) (width 0.2) (layer "F.Cu") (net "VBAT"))
 (segment (start 55.8622 25.6847) (end 55.8622 26.6008) (width 0.2) (layer "F.Cu") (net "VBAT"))
 (segment (start 56.5133 26.6008) (end 56.8625 26.95) (width 0.15) (layer "F.Cu") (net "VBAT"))
 (segment (start 56.8625 26.95) (end 58.4261 28.5136) (width 0.2) (layer "F.Cu") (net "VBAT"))
 (segment (start 24.2002 47.262) (end 24.0365 47.4257) (width 0.2) (layer "F.Cu") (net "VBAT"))
 (segment (start 56.8625 25.05) (end 56.4969 25.05) (width 0.2) (layer "F.Cu") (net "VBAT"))
 (segment (start 30.9767 36.0854) (end 24.2002 42.8619) (width 0.2) (layer "F.Cu") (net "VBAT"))
 (segment (start 24.0365 47.4257) (end 24.4757 47.4257) (width 0.2) (layer "F.Cu") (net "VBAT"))
 (segment (start 56.4969 25.05) (end 55.8622 25.6847) (width 0.2) (layer "F.Cu") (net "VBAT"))
 (segment (start 67.6591 28.7209) (end 67.5794 28.7209) (width 0.2) (layer "F.Cu") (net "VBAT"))
 (segment (start 56.8625 26.95) (end 47.7271 36.0854) (width 0.2) (layer "F.Cu") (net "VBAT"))
 (segment (start 24.2002 42.8619) (end 24.2002 47.262) (width 0.2) (layer "F.Cu") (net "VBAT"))
 (segment (start 55.8622 26.6008) (end 56.5133 26.6008) (width 0.15) (layer "F.Cu") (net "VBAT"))
 (segment (start 24.4757 47.4257) (end 25.05 48) (width 0.2) (layer "F.Cu") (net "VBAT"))
 (segment (start 58.4261 28.5136) (end 66.2895 28.5136) (width 0.2) (layer "F.Cu") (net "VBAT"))
 (segment (start 68.475 27.905) (end 67.6591 28.7209) (width 0.2) (layer "F.Cu") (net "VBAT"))
 (via (at 66.2895 28.5136) (size 0.6) (drill 0.3) (layers "F.Cu" "B.Cu") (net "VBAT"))
 (via (at 24.0365 47.4257) (size 0.6) (drill 0.3) (layers "F.Cu" "B.Cu") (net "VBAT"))
 (via (at 67.5794 28.7209) (size 0.6) (drill 0.3) (layers "F.Cu" "B.Cu") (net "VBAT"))
 (segment (start 67.5794 28.7209) (end 66.4968 28.7209) (width 0.2) (layer "B.Cu") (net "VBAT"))
 (segment (start 20 56) (end 24.0365 51.9635) (width 0.2) (layer "B.Cu") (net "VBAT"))
 (segment (start 24.0365 51.9635) (end 24.0365 47.4257) (width 0.2) (layer "B.Cu") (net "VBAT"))
 (segment (start 66.4968 28.7209) (end 66.2895 28.5136) (width 0.2) (layer "B.Cu") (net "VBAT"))
 (segment (start 68.475 26.635) (end 66.9691 26.635) (width 0.2) (layer "F.Cu") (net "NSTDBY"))
 (segment (start 66.9691 41.2059) (end 66.9691 26.635) (width 0.2) (layer "F.Cu") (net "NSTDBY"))
 (segment (start 64.175 44) (end 66.9691 41.2059) (width 0.2) (layer "F.Cu") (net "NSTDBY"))
 (via (at 66.9691 26.635) (size 0.6) (drill 0.3) (layers "F.Cu" "B.Cu") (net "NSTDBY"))
 (segment (start 58.4179 43.2571) (end 57.675 44) (width 0.2) (layer "F.Cu") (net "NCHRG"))
 (segment (start 69.1442 26.0342) (end 68.475 25.365) (width 0.15) (layer "F.Cu") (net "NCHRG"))
 (segment (start 70.4089 26.0342) (end 69.1442 26.0342) (width 0.15) (layer "F.Cu") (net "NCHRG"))
 (via (at 58.4179 43.2571) (size 0.6) (drill 0.3) (layers "F.Cu" "B.Cu") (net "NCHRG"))
 (via (at 70.4089 26.0342) (size 0.6) (drill 0.3) (layers "F.Cu" "B.Cu") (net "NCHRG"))
 (segment (start 70.4089 31.2661) (end 58.4179 43.2571) (width 0.2) (layer "B.Cu") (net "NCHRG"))
 (segment (start 70.4089 26.0342) (end 70.4089 31.2661) (width 0.2) (layer "B.Cu") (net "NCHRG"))
 (segment (start 61.3516 44.8261) (end 60.2733 43.7478) (width 0.2) (layer "F.Cu") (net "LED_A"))
 (segment (start 29.2125 27.0014) (end 29.2125 26) (width 0.2) (layer "F.Cu") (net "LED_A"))
 (segment (start 64.9989 44.8261) (end 61.3516 44.8261) (width 0.2) (layer "F.Cu") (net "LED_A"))
 (segment (start 59.5772 43.7478) (end 59.5772 43.5629) (width 0.2) (layer "F.Cu") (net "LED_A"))
 (segment (start 59.5772 43.7478) (end 59.325 44) (width 0.2) (layer "F.Cu") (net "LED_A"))
 (segment (start 59.5772 43.5629) (end 52.7844 36.7701) (width 0.2) (layer "F.Cu") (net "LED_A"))
 (segment (start 60.2733 43.7478) (end 59.5772 43.7478) (width 0.2) (layer "F.Cu") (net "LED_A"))
 (segment (start 65.825 44) (end 64.9989 44.8261) (width 0.2) (layer "F.Cu") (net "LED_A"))
 (segment (start 52.7844 36.7701) (end 31.1479 36.7701) (width 0.2) (layer "F.Cu") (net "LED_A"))
 (via (at 29.2125 27.0014) (size 0.6) (drill 0.3) (layers "F.Cu" "B.Cu") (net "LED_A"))
 (via (at 60.2733 43.7478) (size 0.6) (drill 0.3) (layers "F.Cu" "B.Cu") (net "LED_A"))
 (via (at 31.1479 36.7701) (size 0.6) (drill 0.3) (layers "F.Cu" "B.Cu") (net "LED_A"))
 (segment (start 29.2125 27.0014) (end 31.1479 28.9368) (width 0.2) (layer "B.Cu") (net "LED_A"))
 (segment (start 31.1479 28.9368) (end 31.1479 36.7701) (width 0.2) (layer "B.Cu") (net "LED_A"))
 (segment (start 34.0447 22.2498) (end 33.0265 22.2498) (width 0.15) (layer "F.Cu") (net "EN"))
 (segment (start 34.2346 44.3056) (end 33.6306 44.3056) (width 0.2) (layer "F.Cu") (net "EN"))
 (segment (start 31.25 21.5) (end 32.2767 21.5) (width 0.15) (layer "F.Cu") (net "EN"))
 (segment (start 33.6306 44.3056) (end 33.325 44) (width 0.2) (layer "F.Cu") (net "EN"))
 (segment (start 33.0265 22.2498) (end 32.2767 21.5) (width 0.15) (layer "F.Cu") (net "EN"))
 (via (at 34.0447 22.2498) (size 0.6) (drill 0.3) (layers "F.Cu" "B.Cu") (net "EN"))
 (via (at 34.2346 44.3056) (size 0.6) (drill 0.3) (layers "F.Cu" "B.Cu") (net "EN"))
 (segment (start 34.0447 44.1157) (end 34.2346 44.3056) (width 0.2) (layer "B.Cu") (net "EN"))
 (segment (start 34.0447 22.2498) (end 34.0447 44.1157) (width 0.2) (layer "B.Cu") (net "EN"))
 (segment (start 37.4299 47.2549) (end 34.0512 47.2549) (width 0.2) (layer "F.Cu") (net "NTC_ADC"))
 (segment (start 29.989 22.7657) (end 25.6169 22.7657) (width 0.15) (layer "F.Cu") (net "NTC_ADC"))
 (segment (start 31.25 23) (end 30.2233 23) (width 0.15) (layer "F.Cu") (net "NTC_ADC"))
 (segment (start 38.175 48) (end 37.4299 47.2549) (width 0.2) (layer "F.Cu") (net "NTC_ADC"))
 (segment (start 30.2233 23) (end 29.989 22.7657) (width 0.15) (layer "F.Cu") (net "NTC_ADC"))
 (via (at 34.0512 47.2549) (size 0.6) (drill 0.3) (layers "F.Cu" "B.Cu") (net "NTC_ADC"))
 (via (at 25.6169 22.7657) (size 0.6) (drill 0.3) (layers "F.Cu" "B.Cu") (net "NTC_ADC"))
 (segment (start 25.6169 10.8134) (end 25.6169 10.5303) (width 0.15) (layer "B.Cu") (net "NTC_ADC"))
 (segment (start 30.6081 35.3794) (end 27.8266 38.1609) (width 0.2) (layer "B.Cu") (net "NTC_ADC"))
 (segment (start 27.8266 45.0831) (end 29.9984 47.2549) (width 0.2) (layer "B.Cu") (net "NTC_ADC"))
 (segment (start 27.8266 38.1609) (end 27.8266 45.0831) (width 0.2) (layer "B.Cu") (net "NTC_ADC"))
 (segment (start 24.3525 9.1517) (end 24 9.1517) (width 0.2) (layer "B.Cu") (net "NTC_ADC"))
 (segment (start 25.6169 22.7657) (end 25.6169 24.3121) (width 0.2) (layer "B.Cu") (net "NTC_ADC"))
 (segment (start 29.9984 47.2549) (end 34.0512 47.2549) (width 0.2) (layer "B.Cu") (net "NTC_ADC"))
 (segment (start 25.6169 10.8134) (end 25.6169 22.7657) (width 0.2) (layer "B.Cu") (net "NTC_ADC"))
 (segment (start 24 8) (end 24 9.1517) (width 0.2) (layer "B.Cu") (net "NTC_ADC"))
 (segment (start 25.6169 10.5303) (end 25.4996 10.413) (width 0.15) (layer "B.Cu") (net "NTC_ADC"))
 (segment (start 25.4996 10.2988) (end 24.3525 9.1517) (width 0.2) (layer "B.Cu") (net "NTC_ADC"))
 (segment (start 30.6081 29.3033) (end 30.6081 35.3794) (width 0.2) (layer "B.Cu") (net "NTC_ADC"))
 (segment (start 25.6169 24.3121) (end 30.6081 29.3033) (width 0.2) (layer "B.Cu") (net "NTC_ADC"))
 (segment (start 25.4996 10.413) (end 25.4996 10.2988) (width 0.2) (layer "B.Cu") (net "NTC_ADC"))
 (segment (start 26.0902 43.2652) (end 26.825 44) (width 0.2) (layer "F.Cu") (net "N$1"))
 (segment (start 11.2125 26.9777) (end 21.0026 36.7678) (width 0.2) (layer "F.Cu") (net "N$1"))
 (segment (start 21.0026 36.7678) (end 26.0902 36.7678) (width 0.2) (layer "F.Cu") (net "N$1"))
 (segment (start 11.2125 26.9777) (end 11.2125 26) (width 0.2) (layer "F.Cu") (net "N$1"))
 (via (at 11.2125 26.9777) (size 0.6) (drill 0.3) (layers "F.Cu" "B.Cu") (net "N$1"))
 (via (at 26.0902 36.7678) (size 0.6) (drill 0.3) (layers "F.Cu" "B.Cu") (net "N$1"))
 (via (at 26.0902 43.2652) (size 0.6) (drill 0.3) (layers "F.Cu" "B.Cu") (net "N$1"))
 (segment (start 26.0902 43.2652) (end 26.0902 36.7678) (width 0.2) (layer "B.Cu") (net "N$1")))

